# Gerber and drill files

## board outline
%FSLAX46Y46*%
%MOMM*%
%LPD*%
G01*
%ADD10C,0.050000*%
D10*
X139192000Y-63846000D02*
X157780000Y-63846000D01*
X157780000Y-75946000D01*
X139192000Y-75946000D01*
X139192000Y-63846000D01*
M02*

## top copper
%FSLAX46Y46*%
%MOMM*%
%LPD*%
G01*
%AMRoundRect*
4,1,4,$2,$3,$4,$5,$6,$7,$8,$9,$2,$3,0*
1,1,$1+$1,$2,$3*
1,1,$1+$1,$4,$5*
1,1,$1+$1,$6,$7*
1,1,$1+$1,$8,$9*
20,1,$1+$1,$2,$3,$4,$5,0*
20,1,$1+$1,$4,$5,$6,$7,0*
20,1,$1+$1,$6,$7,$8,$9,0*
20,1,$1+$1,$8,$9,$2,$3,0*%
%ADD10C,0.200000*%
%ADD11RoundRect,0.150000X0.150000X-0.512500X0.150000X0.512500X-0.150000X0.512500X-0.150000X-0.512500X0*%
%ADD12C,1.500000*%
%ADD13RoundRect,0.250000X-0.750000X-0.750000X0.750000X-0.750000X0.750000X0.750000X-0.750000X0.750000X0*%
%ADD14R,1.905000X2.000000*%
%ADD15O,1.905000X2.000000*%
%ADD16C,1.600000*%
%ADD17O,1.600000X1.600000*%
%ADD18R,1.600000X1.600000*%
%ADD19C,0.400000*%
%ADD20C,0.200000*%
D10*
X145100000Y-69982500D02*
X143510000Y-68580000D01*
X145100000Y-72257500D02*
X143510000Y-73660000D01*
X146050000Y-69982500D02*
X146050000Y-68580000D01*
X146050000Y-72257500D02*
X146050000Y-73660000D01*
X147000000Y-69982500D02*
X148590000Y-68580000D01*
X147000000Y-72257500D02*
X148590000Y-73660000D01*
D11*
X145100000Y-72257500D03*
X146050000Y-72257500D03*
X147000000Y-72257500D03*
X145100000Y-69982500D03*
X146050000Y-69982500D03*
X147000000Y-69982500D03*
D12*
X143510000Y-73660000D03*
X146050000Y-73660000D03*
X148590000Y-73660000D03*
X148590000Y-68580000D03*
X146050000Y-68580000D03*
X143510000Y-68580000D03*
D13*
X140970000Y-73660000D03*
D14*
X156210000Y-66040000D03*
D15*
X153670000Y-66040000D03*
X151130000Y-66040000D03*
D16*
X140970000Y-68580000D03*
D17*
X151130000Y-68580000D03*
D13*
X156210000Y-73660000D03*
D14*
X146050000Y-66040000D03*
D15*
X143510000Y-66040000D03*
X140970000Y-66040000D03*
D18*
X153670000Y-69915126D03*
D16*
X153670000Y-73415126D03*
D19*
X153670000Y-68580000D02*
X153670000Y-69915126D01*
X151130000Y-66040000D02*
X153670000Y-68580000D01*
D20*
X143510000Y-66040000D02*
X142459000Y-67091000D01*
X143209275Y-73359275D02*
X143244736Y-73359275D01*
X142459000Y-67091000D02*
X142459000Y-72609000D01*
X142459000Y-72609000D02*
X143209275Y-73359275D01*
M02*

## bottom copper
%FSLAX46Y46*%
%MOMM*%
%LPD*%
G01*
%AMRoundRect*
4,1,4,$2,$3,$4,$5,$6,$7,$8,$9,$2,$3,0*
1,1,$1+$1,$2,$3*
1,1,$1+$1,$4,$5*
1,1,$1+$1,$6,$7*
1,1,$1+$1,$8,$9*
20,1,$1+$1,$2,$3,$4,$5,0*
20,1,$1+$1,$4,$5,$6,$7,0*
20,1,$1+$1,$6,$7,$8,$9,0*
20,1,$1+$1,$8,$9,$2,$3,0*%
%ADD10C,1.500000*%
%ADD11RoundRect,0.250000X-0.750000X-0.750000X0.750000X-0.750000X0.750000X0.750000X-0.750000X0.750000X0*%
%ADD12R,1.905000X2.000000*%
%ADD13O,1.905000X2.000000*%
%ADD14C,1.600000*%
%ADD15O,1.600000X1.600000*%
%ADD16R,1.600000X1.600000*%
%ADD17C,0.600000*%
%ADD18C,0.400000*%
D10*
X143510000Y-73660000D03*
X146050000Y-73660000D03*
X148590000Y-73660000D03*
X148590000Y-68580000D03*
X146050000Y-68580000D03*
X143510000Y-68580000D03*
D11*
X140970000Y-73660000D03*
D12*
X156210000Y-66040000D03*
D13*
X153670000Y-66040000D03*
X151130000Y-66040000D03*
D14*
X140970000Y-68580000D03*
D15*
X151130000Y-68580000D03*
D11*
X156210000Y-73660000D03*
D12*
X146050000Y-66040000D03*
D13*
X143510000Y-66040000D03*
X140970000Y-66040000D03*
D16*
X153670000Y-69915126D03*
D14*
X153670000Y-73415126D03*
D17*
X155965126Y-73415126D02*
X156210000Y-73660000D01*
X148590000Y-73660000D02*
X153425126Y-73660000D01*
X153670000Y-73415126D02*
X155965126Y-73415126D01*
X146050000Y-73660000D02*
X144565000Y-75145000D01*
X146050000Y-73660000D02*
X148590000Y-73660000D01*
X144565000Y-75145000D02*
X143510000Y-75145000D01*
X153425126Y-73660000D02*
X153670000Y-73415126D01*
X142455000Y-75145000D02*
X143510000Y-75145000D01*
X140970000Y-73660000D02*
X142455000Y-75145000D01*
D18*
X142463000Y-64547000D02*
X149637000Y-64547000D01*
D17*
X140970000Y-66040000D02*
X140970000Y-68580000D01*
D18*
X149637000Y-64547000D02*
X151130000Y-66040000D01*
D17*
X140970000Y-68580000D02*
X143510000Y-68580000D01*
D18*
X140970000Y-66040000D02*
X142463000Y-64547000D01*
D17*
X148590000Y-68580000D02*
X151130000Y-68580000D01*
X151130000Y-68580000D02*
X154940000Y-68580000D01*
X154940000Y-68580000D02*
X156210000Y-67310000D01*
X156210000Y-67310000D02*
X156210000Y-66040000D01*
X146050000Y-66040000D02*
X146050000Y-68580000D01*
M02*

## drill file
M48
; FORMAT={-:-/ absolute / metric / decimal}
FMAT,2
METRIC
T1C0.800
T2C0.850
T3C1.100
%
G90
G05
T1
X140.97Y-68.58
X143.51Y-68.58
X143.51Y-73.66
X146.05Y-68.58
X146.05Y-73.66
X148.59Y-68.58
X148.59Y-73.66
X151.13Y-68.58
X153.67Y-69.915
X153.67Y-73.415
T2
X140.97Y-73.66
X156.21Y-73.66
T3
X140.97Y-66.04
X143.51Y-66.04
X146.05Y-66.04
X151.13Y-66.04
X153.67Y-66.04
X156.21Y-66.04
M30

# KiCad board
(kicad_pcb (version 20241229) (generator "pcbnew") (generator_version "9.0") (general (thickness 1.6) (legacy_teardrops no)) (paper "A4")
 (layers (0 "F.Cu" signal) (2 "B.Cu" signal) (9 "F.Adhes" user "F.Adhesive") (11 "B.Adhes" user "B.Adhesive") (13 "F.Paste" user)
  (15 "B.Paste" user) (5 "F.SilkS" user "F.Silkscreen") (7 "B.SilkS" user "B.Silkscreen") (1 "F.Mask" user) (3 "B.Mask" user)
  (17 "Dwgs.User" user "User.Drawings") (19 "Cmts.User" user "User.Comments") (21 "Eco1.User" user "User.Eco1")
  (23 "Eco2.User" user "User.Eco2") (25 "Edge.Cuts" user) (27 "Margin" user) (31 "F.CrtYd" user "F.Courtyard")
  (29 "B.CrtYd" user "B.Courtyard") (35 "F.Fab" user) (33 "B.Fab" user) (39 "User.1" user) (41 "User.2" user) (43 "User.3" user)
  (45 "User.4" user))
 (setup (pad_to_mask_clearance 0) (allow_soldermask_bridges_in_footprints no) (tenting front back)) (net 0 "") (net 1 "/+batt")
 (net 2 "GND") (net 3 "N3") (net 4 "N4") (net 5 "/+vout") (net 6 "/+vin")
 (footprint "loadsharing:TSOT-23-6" (layer "F.Cu") (at 146.05 71.12 90)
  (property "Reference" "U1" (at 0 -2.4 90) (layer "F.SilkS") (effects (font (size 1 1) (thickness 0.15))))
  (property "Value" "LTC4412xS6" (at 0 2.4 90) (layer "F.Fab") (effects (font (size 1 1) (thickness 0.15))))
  (fp_line (start 1.1375 -0.95) (end 2.54 -2.54) (stroke (width 0.2) (type default)) (layer "F.Cu"))
  (fp_line (start -1.1375 -0.95) (end -2.54 -2.54) (stroke (width 0.2) (type default)) (layer "F.Cu"))
  (fp_line (start 1.1375 0) (end 2.54 0) (stroke (width 0.2) (type default)) (layer "F.Cu"))
  (fp_line (start -1.1375 0) (end -2.54 0) (stroke (width 0.2) (type default)) (layer "F.Cu"))
  (fp_line (start 1.1375 0.95) (end 2.54 2.54) (stroke (width 0.2) (type default)) (layer "F.Cu"))
  (fp_line (start -1.1375 0.95) (end -2.54 2.54) (stroke (width 0.2) (type default)) (layer "F.Cu"))
  (pad "" smd roundrect (at -1.1375 -0.95 90) (size 1.325 0.6) (layers "F.Cu" "F.Mask" "F.Paste") (roundrect_rratio 0.25))
  (pad "" smd roundrect (at -1.1375 0 90) (size 1.325 0.6) (layers "F.Cu" "F.Mask" "F.Paste") (roundrect_rratio 0.25))
  (pad "" smd roundrect (at -1.1375 0.95 90) (size 1.325 0.6) (layers "F.Cu" "F.Mask" "F.Paste") (roundrect_rratio 0.25))
  (pad "" smd roundrect (at 1.1375 -0.95 90) (size 1.325 0.6) (layers "F.Cu" "F.Mask" "F.Paste") (roundrect_rratio 0.25))
  (pad "" smd roundrect (at 1.1375 0 90) (size 1.325 0.6) (layers "F.Cu" "F.Mask" "F.Paste") (roundrect_rratio 0.25))
  (pad "" smd roundrect (at 1.1375 0.95 90) (size 1.325 0.6) (layers "F.Cu" "F.Mask" "F.Paste") (roundrect_rratio 0.25))
  (pad "1" thru_hole circle (at -2.54 -2.54 90) (size 1.5 1.5) (drill 0.8) (layers "*.Cu" "F.Mask" "F.Paste") (remove_unused_layers no)
   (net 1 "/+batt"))
  (pad "2" thru_hole circle (at -2.54 0 90) (size 1.5 1.5) (drill 0.8) (layers "*.Cu" "F.Mask" "F.Paste") (remove_unused_layers no)
   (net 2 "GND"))
  (pad "3" thru_hole circle (at -2.54 2.54 90) (size 1.5 1.5) (drill 0.8) (layers "*.Cu" "F.Mask" "F.Paste") (remove_unused_layers no)
   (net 2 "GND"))
  (pad "4" thru_hole circle (at 2.54 2.54 90) (size 1.5 1.5) (drill 0.8) (layers "*.Cu" "F.Mask" "F.Paste") (remove_unused_layers no)
   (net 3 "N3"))
  (pad "5" thru_hole circle (at 2.54 0 90) (size 1.5 1.5) (drill 0.8) (layers "*.Cu" "F.Mask" "F.Paste") (remove_unused_layers no)
   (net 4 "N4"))
  (pad "6" thru_hole circle (at 2.54 -2.54 90) (size 1.5 1.5) (drill 0.8) (layers "*.Cu" "F.Mask" "F.Paste") (remove_unused_layers no)
   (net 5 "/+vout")))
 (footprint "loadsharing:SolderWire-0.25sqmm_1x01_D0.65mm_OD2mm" (layer "F.Cu") (at 140.97 73.66)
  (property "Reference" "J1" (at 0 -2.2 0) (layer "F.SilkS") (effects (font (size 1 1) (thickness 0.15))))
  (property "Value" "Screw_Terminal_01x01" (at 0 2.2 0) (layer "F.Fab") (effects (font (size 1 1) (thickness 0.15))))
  (pad "1" thru_hole roundrect (at 0 0) (size 2 2) (drill 0.85) (layers "*.Cu" "*.Mask") (remove_unused_layers no) (roundrect_rratio 0.125)
   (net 2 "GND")))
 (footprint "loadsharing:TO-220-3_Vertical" (layer "F.Cu") (at 156.21 66.04 180)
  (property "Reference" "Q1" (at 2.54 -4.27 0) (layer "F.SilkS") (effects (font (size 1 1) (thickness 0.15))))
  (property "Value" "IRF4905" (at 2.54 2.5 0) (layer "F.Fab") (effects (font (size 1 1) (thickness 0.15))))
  (pad "1" thru_hole rect (at 0 0 180) (size 1.905 2) (drill 1.1) (layers "*.Cu" "*.Mask") (remove_unused_layers no) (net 3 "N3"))
  (pad "2" thru_hole oval (at 2.54 0 180) (size 1.905 2) (drill 1.1) (layers "*.Cu" "*.Mask") (remove_unused_layers no) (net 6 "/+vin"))
  (pad "3" thru_hole oval (at 5.08 0 180) (size 1.905 2) (drill 1.1) (layers "*.Cu" "*.Mask") (remove_unused_layers no) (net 5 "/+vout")))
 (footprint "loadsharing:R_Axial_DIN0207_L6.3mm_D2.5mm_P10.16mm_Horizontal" (layer "F.Cu") (at 140.97 68.58)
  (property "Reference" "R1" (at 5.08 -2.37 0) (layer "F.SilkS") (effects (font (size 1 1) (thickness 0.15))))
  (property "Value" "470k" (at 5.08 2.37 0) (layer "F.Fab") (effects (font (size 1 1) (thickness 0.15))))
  (pad "1" thru_hole circle (at 0 0) (size 1.6 1.6) (drill 0.8) (layers "*.Cu" "*.Mask") (remove_unused_layers no) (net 5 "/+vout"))
  (pad "2" thru_hole oval (at 10.16 0) (size 1.6 1.6) (drill 0.8) (layers "*.Cu" "*.Mask") (remove_unused_layers no) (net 3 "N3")))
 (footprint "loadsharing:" (layer "F.Cu") (at 156.21 73.66)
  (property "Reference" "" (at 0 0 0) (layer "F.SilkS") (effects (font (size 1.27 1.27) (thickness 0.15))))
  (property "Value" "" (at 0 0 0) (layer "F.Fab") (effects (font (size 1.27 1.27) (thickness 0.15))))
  (pad "1" thru_hole roundrect (at 0 0) (size 2 2) (drill 0.85) (layers "*.Cu" "*.Mask") (remove_unused_layers no) (roundrect_rratio 0.125)
   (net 2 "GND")))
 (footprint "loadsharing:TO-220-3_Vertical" (layer "F.Cu") (at 146.05 66.04 180)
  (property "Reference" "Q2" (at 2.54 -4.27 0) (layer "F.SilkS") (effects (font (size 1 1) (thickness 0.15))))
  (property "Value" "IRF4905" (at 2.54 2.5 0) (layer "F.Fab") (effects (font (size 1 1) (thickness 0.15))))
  (pad "1" thru_hole rect (at 0 0 180) (size 1.905 2) (drill 1.1) (layers "*.Cu" "*.Mask") (remove_unused_layers no) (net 4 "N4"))
  (pad "2" thru_hole oval (at 2.54 0 180) (size 1.905 2) (drill 1.1) (layers "*.Cu" "*.Mask") (remove_unused_layers no) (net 1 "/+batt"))
  (pad "3" thru_hole oval (at 5.08 0 180) (size 1.905 2) (drill 1.1) (layers "*.Cu" "*.Mask") (remove_unused_layers no) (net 5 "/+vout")))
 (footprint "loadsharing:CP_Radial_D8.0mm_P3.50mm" (layer "F.Cu") (at 153.67 69.915126 -90)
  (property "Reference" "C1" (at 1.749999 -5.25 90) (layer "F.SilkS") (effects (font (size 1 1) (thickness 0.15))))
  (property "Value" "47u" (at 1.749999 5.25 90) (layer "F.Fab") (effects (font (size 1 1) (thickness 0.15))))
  (pad "1" thru_hole rect (at 0 0 270) (size 1.6 1.6) (drill 0.8) (layers "*.Cu" "*.Mask") (remove_unused_layers no) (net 5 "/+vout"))
  (pad "2" thru_hole circle (at 3.5 0 270) (size 1.6 1.6) (drill 0.8) (layers "*.Cu" "*.Mask") (remove_unused_layers no) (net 2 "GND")))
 (gr_rect (start 139.192 63.846) (end 157.78 75.946) (stroke (width 0.05) (type solid)) (fill no) (layer "Edge.Cuts"))
 (segment (start 155.965126 73.415126) (end 156.21 73.66) (width 0.6) (layer "B.Cu") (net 2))
 (segment (start 148.59 73.66) (end 153.425126 73.66) (width 0.6) (layer "B.Cu") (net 2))
 (segment (start 153.67 73.415126) (end 155.965126 73.415126) (width 0.6) (layer "B.Cu") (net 2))
 (segment (start 146.05 73.66) (end 144.565 75.145) (width 0.6) (layer "B.Cu") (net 2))
 (segment (start 146.05 73.66) (end 148.59 73.66) (width 0.6) (layer "B.Cu") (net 2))
 (segment (start 144.565 75.145) (end 143.51 75.145) (width 0.6) (layer "B.Cu") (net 2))
 (segment (start 153.425126 73.66) (end 153.67 73.415126) (width 0.6) (layer "B.Cu") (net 2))
 (segment (start 142.455 75.145) (end 143.51 75.145) (width 0.6) (layer "B.Cu") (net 2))
 (segment (start 140.97 73.66) (end 142.455 75.145) (width 0.6) (layer "B.Cu") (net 2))
 (segment (start 153.67 68.58) (end 153.67 69.915126) (width 0.4) (layer "F.Cu") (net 5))
 (segment (start 151.13 66.04) (end 153.67 68.58) (width 0.4) (layer "F.Cu") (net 5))
 (segment (start 142.463 64.547) (end 149.637 64.547) (width 0.4) (layer "B.Cu") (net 5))
 (segment (start 140.97 66.04) (end 140.97 68.58) (width 0.6) (layer "B.Cu") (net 5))
 (segment (start 149.637 64.547) (end 151.13 66.04) (width 0.4) (layer "B.Cu") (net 5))
 (segment (start 140.97 68.58) (end 143.51 68.58) (width 0.6) (layer "B.Cu") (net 5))
 (segment (start 140.97 66.04) (end 142.463 64.547) (width 0.4) (layer "B.Cu") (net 5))
 (segment (start 148.59 68.58) (end 151.13 68.58) (width 0.6) (layer "B.Cu") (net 3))
 (segment (start 151.13 68.58) (end 154.94 68.58) (width 0.6) (layer "B.Cu") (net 3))
 (segment (start 154.94 68.58) (end 156.21 67.31) (width 0.6) (layer "B.Cu") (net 3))
 (segment (start 156.21 67.31) (end 156.21 66.04) (width 0.6) (layer "B.Cu") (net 3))
 (segment (start 146.05 66.04) (end 146.05 68.58) (width 0.6) (layer "B.Cu") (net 4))
 (segment (start 143.51 66.04) (end 142.459 67.091) (width 0.2) (layer "F.Cu") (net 1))
 (segment (start 143.209275 73.359275) (end 143.244736 73.359275) (width 0.2) (layer "F.Cu") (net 1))
 (segment (start 142.459 67.091) (end 142.459 72.609) (width 0.2) (layer "F.Cu") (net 1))
 (segment (start 142.459 72.609) (end 143.209275 73.359275) (width 0.2) (layer "F.Cu") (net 1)))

